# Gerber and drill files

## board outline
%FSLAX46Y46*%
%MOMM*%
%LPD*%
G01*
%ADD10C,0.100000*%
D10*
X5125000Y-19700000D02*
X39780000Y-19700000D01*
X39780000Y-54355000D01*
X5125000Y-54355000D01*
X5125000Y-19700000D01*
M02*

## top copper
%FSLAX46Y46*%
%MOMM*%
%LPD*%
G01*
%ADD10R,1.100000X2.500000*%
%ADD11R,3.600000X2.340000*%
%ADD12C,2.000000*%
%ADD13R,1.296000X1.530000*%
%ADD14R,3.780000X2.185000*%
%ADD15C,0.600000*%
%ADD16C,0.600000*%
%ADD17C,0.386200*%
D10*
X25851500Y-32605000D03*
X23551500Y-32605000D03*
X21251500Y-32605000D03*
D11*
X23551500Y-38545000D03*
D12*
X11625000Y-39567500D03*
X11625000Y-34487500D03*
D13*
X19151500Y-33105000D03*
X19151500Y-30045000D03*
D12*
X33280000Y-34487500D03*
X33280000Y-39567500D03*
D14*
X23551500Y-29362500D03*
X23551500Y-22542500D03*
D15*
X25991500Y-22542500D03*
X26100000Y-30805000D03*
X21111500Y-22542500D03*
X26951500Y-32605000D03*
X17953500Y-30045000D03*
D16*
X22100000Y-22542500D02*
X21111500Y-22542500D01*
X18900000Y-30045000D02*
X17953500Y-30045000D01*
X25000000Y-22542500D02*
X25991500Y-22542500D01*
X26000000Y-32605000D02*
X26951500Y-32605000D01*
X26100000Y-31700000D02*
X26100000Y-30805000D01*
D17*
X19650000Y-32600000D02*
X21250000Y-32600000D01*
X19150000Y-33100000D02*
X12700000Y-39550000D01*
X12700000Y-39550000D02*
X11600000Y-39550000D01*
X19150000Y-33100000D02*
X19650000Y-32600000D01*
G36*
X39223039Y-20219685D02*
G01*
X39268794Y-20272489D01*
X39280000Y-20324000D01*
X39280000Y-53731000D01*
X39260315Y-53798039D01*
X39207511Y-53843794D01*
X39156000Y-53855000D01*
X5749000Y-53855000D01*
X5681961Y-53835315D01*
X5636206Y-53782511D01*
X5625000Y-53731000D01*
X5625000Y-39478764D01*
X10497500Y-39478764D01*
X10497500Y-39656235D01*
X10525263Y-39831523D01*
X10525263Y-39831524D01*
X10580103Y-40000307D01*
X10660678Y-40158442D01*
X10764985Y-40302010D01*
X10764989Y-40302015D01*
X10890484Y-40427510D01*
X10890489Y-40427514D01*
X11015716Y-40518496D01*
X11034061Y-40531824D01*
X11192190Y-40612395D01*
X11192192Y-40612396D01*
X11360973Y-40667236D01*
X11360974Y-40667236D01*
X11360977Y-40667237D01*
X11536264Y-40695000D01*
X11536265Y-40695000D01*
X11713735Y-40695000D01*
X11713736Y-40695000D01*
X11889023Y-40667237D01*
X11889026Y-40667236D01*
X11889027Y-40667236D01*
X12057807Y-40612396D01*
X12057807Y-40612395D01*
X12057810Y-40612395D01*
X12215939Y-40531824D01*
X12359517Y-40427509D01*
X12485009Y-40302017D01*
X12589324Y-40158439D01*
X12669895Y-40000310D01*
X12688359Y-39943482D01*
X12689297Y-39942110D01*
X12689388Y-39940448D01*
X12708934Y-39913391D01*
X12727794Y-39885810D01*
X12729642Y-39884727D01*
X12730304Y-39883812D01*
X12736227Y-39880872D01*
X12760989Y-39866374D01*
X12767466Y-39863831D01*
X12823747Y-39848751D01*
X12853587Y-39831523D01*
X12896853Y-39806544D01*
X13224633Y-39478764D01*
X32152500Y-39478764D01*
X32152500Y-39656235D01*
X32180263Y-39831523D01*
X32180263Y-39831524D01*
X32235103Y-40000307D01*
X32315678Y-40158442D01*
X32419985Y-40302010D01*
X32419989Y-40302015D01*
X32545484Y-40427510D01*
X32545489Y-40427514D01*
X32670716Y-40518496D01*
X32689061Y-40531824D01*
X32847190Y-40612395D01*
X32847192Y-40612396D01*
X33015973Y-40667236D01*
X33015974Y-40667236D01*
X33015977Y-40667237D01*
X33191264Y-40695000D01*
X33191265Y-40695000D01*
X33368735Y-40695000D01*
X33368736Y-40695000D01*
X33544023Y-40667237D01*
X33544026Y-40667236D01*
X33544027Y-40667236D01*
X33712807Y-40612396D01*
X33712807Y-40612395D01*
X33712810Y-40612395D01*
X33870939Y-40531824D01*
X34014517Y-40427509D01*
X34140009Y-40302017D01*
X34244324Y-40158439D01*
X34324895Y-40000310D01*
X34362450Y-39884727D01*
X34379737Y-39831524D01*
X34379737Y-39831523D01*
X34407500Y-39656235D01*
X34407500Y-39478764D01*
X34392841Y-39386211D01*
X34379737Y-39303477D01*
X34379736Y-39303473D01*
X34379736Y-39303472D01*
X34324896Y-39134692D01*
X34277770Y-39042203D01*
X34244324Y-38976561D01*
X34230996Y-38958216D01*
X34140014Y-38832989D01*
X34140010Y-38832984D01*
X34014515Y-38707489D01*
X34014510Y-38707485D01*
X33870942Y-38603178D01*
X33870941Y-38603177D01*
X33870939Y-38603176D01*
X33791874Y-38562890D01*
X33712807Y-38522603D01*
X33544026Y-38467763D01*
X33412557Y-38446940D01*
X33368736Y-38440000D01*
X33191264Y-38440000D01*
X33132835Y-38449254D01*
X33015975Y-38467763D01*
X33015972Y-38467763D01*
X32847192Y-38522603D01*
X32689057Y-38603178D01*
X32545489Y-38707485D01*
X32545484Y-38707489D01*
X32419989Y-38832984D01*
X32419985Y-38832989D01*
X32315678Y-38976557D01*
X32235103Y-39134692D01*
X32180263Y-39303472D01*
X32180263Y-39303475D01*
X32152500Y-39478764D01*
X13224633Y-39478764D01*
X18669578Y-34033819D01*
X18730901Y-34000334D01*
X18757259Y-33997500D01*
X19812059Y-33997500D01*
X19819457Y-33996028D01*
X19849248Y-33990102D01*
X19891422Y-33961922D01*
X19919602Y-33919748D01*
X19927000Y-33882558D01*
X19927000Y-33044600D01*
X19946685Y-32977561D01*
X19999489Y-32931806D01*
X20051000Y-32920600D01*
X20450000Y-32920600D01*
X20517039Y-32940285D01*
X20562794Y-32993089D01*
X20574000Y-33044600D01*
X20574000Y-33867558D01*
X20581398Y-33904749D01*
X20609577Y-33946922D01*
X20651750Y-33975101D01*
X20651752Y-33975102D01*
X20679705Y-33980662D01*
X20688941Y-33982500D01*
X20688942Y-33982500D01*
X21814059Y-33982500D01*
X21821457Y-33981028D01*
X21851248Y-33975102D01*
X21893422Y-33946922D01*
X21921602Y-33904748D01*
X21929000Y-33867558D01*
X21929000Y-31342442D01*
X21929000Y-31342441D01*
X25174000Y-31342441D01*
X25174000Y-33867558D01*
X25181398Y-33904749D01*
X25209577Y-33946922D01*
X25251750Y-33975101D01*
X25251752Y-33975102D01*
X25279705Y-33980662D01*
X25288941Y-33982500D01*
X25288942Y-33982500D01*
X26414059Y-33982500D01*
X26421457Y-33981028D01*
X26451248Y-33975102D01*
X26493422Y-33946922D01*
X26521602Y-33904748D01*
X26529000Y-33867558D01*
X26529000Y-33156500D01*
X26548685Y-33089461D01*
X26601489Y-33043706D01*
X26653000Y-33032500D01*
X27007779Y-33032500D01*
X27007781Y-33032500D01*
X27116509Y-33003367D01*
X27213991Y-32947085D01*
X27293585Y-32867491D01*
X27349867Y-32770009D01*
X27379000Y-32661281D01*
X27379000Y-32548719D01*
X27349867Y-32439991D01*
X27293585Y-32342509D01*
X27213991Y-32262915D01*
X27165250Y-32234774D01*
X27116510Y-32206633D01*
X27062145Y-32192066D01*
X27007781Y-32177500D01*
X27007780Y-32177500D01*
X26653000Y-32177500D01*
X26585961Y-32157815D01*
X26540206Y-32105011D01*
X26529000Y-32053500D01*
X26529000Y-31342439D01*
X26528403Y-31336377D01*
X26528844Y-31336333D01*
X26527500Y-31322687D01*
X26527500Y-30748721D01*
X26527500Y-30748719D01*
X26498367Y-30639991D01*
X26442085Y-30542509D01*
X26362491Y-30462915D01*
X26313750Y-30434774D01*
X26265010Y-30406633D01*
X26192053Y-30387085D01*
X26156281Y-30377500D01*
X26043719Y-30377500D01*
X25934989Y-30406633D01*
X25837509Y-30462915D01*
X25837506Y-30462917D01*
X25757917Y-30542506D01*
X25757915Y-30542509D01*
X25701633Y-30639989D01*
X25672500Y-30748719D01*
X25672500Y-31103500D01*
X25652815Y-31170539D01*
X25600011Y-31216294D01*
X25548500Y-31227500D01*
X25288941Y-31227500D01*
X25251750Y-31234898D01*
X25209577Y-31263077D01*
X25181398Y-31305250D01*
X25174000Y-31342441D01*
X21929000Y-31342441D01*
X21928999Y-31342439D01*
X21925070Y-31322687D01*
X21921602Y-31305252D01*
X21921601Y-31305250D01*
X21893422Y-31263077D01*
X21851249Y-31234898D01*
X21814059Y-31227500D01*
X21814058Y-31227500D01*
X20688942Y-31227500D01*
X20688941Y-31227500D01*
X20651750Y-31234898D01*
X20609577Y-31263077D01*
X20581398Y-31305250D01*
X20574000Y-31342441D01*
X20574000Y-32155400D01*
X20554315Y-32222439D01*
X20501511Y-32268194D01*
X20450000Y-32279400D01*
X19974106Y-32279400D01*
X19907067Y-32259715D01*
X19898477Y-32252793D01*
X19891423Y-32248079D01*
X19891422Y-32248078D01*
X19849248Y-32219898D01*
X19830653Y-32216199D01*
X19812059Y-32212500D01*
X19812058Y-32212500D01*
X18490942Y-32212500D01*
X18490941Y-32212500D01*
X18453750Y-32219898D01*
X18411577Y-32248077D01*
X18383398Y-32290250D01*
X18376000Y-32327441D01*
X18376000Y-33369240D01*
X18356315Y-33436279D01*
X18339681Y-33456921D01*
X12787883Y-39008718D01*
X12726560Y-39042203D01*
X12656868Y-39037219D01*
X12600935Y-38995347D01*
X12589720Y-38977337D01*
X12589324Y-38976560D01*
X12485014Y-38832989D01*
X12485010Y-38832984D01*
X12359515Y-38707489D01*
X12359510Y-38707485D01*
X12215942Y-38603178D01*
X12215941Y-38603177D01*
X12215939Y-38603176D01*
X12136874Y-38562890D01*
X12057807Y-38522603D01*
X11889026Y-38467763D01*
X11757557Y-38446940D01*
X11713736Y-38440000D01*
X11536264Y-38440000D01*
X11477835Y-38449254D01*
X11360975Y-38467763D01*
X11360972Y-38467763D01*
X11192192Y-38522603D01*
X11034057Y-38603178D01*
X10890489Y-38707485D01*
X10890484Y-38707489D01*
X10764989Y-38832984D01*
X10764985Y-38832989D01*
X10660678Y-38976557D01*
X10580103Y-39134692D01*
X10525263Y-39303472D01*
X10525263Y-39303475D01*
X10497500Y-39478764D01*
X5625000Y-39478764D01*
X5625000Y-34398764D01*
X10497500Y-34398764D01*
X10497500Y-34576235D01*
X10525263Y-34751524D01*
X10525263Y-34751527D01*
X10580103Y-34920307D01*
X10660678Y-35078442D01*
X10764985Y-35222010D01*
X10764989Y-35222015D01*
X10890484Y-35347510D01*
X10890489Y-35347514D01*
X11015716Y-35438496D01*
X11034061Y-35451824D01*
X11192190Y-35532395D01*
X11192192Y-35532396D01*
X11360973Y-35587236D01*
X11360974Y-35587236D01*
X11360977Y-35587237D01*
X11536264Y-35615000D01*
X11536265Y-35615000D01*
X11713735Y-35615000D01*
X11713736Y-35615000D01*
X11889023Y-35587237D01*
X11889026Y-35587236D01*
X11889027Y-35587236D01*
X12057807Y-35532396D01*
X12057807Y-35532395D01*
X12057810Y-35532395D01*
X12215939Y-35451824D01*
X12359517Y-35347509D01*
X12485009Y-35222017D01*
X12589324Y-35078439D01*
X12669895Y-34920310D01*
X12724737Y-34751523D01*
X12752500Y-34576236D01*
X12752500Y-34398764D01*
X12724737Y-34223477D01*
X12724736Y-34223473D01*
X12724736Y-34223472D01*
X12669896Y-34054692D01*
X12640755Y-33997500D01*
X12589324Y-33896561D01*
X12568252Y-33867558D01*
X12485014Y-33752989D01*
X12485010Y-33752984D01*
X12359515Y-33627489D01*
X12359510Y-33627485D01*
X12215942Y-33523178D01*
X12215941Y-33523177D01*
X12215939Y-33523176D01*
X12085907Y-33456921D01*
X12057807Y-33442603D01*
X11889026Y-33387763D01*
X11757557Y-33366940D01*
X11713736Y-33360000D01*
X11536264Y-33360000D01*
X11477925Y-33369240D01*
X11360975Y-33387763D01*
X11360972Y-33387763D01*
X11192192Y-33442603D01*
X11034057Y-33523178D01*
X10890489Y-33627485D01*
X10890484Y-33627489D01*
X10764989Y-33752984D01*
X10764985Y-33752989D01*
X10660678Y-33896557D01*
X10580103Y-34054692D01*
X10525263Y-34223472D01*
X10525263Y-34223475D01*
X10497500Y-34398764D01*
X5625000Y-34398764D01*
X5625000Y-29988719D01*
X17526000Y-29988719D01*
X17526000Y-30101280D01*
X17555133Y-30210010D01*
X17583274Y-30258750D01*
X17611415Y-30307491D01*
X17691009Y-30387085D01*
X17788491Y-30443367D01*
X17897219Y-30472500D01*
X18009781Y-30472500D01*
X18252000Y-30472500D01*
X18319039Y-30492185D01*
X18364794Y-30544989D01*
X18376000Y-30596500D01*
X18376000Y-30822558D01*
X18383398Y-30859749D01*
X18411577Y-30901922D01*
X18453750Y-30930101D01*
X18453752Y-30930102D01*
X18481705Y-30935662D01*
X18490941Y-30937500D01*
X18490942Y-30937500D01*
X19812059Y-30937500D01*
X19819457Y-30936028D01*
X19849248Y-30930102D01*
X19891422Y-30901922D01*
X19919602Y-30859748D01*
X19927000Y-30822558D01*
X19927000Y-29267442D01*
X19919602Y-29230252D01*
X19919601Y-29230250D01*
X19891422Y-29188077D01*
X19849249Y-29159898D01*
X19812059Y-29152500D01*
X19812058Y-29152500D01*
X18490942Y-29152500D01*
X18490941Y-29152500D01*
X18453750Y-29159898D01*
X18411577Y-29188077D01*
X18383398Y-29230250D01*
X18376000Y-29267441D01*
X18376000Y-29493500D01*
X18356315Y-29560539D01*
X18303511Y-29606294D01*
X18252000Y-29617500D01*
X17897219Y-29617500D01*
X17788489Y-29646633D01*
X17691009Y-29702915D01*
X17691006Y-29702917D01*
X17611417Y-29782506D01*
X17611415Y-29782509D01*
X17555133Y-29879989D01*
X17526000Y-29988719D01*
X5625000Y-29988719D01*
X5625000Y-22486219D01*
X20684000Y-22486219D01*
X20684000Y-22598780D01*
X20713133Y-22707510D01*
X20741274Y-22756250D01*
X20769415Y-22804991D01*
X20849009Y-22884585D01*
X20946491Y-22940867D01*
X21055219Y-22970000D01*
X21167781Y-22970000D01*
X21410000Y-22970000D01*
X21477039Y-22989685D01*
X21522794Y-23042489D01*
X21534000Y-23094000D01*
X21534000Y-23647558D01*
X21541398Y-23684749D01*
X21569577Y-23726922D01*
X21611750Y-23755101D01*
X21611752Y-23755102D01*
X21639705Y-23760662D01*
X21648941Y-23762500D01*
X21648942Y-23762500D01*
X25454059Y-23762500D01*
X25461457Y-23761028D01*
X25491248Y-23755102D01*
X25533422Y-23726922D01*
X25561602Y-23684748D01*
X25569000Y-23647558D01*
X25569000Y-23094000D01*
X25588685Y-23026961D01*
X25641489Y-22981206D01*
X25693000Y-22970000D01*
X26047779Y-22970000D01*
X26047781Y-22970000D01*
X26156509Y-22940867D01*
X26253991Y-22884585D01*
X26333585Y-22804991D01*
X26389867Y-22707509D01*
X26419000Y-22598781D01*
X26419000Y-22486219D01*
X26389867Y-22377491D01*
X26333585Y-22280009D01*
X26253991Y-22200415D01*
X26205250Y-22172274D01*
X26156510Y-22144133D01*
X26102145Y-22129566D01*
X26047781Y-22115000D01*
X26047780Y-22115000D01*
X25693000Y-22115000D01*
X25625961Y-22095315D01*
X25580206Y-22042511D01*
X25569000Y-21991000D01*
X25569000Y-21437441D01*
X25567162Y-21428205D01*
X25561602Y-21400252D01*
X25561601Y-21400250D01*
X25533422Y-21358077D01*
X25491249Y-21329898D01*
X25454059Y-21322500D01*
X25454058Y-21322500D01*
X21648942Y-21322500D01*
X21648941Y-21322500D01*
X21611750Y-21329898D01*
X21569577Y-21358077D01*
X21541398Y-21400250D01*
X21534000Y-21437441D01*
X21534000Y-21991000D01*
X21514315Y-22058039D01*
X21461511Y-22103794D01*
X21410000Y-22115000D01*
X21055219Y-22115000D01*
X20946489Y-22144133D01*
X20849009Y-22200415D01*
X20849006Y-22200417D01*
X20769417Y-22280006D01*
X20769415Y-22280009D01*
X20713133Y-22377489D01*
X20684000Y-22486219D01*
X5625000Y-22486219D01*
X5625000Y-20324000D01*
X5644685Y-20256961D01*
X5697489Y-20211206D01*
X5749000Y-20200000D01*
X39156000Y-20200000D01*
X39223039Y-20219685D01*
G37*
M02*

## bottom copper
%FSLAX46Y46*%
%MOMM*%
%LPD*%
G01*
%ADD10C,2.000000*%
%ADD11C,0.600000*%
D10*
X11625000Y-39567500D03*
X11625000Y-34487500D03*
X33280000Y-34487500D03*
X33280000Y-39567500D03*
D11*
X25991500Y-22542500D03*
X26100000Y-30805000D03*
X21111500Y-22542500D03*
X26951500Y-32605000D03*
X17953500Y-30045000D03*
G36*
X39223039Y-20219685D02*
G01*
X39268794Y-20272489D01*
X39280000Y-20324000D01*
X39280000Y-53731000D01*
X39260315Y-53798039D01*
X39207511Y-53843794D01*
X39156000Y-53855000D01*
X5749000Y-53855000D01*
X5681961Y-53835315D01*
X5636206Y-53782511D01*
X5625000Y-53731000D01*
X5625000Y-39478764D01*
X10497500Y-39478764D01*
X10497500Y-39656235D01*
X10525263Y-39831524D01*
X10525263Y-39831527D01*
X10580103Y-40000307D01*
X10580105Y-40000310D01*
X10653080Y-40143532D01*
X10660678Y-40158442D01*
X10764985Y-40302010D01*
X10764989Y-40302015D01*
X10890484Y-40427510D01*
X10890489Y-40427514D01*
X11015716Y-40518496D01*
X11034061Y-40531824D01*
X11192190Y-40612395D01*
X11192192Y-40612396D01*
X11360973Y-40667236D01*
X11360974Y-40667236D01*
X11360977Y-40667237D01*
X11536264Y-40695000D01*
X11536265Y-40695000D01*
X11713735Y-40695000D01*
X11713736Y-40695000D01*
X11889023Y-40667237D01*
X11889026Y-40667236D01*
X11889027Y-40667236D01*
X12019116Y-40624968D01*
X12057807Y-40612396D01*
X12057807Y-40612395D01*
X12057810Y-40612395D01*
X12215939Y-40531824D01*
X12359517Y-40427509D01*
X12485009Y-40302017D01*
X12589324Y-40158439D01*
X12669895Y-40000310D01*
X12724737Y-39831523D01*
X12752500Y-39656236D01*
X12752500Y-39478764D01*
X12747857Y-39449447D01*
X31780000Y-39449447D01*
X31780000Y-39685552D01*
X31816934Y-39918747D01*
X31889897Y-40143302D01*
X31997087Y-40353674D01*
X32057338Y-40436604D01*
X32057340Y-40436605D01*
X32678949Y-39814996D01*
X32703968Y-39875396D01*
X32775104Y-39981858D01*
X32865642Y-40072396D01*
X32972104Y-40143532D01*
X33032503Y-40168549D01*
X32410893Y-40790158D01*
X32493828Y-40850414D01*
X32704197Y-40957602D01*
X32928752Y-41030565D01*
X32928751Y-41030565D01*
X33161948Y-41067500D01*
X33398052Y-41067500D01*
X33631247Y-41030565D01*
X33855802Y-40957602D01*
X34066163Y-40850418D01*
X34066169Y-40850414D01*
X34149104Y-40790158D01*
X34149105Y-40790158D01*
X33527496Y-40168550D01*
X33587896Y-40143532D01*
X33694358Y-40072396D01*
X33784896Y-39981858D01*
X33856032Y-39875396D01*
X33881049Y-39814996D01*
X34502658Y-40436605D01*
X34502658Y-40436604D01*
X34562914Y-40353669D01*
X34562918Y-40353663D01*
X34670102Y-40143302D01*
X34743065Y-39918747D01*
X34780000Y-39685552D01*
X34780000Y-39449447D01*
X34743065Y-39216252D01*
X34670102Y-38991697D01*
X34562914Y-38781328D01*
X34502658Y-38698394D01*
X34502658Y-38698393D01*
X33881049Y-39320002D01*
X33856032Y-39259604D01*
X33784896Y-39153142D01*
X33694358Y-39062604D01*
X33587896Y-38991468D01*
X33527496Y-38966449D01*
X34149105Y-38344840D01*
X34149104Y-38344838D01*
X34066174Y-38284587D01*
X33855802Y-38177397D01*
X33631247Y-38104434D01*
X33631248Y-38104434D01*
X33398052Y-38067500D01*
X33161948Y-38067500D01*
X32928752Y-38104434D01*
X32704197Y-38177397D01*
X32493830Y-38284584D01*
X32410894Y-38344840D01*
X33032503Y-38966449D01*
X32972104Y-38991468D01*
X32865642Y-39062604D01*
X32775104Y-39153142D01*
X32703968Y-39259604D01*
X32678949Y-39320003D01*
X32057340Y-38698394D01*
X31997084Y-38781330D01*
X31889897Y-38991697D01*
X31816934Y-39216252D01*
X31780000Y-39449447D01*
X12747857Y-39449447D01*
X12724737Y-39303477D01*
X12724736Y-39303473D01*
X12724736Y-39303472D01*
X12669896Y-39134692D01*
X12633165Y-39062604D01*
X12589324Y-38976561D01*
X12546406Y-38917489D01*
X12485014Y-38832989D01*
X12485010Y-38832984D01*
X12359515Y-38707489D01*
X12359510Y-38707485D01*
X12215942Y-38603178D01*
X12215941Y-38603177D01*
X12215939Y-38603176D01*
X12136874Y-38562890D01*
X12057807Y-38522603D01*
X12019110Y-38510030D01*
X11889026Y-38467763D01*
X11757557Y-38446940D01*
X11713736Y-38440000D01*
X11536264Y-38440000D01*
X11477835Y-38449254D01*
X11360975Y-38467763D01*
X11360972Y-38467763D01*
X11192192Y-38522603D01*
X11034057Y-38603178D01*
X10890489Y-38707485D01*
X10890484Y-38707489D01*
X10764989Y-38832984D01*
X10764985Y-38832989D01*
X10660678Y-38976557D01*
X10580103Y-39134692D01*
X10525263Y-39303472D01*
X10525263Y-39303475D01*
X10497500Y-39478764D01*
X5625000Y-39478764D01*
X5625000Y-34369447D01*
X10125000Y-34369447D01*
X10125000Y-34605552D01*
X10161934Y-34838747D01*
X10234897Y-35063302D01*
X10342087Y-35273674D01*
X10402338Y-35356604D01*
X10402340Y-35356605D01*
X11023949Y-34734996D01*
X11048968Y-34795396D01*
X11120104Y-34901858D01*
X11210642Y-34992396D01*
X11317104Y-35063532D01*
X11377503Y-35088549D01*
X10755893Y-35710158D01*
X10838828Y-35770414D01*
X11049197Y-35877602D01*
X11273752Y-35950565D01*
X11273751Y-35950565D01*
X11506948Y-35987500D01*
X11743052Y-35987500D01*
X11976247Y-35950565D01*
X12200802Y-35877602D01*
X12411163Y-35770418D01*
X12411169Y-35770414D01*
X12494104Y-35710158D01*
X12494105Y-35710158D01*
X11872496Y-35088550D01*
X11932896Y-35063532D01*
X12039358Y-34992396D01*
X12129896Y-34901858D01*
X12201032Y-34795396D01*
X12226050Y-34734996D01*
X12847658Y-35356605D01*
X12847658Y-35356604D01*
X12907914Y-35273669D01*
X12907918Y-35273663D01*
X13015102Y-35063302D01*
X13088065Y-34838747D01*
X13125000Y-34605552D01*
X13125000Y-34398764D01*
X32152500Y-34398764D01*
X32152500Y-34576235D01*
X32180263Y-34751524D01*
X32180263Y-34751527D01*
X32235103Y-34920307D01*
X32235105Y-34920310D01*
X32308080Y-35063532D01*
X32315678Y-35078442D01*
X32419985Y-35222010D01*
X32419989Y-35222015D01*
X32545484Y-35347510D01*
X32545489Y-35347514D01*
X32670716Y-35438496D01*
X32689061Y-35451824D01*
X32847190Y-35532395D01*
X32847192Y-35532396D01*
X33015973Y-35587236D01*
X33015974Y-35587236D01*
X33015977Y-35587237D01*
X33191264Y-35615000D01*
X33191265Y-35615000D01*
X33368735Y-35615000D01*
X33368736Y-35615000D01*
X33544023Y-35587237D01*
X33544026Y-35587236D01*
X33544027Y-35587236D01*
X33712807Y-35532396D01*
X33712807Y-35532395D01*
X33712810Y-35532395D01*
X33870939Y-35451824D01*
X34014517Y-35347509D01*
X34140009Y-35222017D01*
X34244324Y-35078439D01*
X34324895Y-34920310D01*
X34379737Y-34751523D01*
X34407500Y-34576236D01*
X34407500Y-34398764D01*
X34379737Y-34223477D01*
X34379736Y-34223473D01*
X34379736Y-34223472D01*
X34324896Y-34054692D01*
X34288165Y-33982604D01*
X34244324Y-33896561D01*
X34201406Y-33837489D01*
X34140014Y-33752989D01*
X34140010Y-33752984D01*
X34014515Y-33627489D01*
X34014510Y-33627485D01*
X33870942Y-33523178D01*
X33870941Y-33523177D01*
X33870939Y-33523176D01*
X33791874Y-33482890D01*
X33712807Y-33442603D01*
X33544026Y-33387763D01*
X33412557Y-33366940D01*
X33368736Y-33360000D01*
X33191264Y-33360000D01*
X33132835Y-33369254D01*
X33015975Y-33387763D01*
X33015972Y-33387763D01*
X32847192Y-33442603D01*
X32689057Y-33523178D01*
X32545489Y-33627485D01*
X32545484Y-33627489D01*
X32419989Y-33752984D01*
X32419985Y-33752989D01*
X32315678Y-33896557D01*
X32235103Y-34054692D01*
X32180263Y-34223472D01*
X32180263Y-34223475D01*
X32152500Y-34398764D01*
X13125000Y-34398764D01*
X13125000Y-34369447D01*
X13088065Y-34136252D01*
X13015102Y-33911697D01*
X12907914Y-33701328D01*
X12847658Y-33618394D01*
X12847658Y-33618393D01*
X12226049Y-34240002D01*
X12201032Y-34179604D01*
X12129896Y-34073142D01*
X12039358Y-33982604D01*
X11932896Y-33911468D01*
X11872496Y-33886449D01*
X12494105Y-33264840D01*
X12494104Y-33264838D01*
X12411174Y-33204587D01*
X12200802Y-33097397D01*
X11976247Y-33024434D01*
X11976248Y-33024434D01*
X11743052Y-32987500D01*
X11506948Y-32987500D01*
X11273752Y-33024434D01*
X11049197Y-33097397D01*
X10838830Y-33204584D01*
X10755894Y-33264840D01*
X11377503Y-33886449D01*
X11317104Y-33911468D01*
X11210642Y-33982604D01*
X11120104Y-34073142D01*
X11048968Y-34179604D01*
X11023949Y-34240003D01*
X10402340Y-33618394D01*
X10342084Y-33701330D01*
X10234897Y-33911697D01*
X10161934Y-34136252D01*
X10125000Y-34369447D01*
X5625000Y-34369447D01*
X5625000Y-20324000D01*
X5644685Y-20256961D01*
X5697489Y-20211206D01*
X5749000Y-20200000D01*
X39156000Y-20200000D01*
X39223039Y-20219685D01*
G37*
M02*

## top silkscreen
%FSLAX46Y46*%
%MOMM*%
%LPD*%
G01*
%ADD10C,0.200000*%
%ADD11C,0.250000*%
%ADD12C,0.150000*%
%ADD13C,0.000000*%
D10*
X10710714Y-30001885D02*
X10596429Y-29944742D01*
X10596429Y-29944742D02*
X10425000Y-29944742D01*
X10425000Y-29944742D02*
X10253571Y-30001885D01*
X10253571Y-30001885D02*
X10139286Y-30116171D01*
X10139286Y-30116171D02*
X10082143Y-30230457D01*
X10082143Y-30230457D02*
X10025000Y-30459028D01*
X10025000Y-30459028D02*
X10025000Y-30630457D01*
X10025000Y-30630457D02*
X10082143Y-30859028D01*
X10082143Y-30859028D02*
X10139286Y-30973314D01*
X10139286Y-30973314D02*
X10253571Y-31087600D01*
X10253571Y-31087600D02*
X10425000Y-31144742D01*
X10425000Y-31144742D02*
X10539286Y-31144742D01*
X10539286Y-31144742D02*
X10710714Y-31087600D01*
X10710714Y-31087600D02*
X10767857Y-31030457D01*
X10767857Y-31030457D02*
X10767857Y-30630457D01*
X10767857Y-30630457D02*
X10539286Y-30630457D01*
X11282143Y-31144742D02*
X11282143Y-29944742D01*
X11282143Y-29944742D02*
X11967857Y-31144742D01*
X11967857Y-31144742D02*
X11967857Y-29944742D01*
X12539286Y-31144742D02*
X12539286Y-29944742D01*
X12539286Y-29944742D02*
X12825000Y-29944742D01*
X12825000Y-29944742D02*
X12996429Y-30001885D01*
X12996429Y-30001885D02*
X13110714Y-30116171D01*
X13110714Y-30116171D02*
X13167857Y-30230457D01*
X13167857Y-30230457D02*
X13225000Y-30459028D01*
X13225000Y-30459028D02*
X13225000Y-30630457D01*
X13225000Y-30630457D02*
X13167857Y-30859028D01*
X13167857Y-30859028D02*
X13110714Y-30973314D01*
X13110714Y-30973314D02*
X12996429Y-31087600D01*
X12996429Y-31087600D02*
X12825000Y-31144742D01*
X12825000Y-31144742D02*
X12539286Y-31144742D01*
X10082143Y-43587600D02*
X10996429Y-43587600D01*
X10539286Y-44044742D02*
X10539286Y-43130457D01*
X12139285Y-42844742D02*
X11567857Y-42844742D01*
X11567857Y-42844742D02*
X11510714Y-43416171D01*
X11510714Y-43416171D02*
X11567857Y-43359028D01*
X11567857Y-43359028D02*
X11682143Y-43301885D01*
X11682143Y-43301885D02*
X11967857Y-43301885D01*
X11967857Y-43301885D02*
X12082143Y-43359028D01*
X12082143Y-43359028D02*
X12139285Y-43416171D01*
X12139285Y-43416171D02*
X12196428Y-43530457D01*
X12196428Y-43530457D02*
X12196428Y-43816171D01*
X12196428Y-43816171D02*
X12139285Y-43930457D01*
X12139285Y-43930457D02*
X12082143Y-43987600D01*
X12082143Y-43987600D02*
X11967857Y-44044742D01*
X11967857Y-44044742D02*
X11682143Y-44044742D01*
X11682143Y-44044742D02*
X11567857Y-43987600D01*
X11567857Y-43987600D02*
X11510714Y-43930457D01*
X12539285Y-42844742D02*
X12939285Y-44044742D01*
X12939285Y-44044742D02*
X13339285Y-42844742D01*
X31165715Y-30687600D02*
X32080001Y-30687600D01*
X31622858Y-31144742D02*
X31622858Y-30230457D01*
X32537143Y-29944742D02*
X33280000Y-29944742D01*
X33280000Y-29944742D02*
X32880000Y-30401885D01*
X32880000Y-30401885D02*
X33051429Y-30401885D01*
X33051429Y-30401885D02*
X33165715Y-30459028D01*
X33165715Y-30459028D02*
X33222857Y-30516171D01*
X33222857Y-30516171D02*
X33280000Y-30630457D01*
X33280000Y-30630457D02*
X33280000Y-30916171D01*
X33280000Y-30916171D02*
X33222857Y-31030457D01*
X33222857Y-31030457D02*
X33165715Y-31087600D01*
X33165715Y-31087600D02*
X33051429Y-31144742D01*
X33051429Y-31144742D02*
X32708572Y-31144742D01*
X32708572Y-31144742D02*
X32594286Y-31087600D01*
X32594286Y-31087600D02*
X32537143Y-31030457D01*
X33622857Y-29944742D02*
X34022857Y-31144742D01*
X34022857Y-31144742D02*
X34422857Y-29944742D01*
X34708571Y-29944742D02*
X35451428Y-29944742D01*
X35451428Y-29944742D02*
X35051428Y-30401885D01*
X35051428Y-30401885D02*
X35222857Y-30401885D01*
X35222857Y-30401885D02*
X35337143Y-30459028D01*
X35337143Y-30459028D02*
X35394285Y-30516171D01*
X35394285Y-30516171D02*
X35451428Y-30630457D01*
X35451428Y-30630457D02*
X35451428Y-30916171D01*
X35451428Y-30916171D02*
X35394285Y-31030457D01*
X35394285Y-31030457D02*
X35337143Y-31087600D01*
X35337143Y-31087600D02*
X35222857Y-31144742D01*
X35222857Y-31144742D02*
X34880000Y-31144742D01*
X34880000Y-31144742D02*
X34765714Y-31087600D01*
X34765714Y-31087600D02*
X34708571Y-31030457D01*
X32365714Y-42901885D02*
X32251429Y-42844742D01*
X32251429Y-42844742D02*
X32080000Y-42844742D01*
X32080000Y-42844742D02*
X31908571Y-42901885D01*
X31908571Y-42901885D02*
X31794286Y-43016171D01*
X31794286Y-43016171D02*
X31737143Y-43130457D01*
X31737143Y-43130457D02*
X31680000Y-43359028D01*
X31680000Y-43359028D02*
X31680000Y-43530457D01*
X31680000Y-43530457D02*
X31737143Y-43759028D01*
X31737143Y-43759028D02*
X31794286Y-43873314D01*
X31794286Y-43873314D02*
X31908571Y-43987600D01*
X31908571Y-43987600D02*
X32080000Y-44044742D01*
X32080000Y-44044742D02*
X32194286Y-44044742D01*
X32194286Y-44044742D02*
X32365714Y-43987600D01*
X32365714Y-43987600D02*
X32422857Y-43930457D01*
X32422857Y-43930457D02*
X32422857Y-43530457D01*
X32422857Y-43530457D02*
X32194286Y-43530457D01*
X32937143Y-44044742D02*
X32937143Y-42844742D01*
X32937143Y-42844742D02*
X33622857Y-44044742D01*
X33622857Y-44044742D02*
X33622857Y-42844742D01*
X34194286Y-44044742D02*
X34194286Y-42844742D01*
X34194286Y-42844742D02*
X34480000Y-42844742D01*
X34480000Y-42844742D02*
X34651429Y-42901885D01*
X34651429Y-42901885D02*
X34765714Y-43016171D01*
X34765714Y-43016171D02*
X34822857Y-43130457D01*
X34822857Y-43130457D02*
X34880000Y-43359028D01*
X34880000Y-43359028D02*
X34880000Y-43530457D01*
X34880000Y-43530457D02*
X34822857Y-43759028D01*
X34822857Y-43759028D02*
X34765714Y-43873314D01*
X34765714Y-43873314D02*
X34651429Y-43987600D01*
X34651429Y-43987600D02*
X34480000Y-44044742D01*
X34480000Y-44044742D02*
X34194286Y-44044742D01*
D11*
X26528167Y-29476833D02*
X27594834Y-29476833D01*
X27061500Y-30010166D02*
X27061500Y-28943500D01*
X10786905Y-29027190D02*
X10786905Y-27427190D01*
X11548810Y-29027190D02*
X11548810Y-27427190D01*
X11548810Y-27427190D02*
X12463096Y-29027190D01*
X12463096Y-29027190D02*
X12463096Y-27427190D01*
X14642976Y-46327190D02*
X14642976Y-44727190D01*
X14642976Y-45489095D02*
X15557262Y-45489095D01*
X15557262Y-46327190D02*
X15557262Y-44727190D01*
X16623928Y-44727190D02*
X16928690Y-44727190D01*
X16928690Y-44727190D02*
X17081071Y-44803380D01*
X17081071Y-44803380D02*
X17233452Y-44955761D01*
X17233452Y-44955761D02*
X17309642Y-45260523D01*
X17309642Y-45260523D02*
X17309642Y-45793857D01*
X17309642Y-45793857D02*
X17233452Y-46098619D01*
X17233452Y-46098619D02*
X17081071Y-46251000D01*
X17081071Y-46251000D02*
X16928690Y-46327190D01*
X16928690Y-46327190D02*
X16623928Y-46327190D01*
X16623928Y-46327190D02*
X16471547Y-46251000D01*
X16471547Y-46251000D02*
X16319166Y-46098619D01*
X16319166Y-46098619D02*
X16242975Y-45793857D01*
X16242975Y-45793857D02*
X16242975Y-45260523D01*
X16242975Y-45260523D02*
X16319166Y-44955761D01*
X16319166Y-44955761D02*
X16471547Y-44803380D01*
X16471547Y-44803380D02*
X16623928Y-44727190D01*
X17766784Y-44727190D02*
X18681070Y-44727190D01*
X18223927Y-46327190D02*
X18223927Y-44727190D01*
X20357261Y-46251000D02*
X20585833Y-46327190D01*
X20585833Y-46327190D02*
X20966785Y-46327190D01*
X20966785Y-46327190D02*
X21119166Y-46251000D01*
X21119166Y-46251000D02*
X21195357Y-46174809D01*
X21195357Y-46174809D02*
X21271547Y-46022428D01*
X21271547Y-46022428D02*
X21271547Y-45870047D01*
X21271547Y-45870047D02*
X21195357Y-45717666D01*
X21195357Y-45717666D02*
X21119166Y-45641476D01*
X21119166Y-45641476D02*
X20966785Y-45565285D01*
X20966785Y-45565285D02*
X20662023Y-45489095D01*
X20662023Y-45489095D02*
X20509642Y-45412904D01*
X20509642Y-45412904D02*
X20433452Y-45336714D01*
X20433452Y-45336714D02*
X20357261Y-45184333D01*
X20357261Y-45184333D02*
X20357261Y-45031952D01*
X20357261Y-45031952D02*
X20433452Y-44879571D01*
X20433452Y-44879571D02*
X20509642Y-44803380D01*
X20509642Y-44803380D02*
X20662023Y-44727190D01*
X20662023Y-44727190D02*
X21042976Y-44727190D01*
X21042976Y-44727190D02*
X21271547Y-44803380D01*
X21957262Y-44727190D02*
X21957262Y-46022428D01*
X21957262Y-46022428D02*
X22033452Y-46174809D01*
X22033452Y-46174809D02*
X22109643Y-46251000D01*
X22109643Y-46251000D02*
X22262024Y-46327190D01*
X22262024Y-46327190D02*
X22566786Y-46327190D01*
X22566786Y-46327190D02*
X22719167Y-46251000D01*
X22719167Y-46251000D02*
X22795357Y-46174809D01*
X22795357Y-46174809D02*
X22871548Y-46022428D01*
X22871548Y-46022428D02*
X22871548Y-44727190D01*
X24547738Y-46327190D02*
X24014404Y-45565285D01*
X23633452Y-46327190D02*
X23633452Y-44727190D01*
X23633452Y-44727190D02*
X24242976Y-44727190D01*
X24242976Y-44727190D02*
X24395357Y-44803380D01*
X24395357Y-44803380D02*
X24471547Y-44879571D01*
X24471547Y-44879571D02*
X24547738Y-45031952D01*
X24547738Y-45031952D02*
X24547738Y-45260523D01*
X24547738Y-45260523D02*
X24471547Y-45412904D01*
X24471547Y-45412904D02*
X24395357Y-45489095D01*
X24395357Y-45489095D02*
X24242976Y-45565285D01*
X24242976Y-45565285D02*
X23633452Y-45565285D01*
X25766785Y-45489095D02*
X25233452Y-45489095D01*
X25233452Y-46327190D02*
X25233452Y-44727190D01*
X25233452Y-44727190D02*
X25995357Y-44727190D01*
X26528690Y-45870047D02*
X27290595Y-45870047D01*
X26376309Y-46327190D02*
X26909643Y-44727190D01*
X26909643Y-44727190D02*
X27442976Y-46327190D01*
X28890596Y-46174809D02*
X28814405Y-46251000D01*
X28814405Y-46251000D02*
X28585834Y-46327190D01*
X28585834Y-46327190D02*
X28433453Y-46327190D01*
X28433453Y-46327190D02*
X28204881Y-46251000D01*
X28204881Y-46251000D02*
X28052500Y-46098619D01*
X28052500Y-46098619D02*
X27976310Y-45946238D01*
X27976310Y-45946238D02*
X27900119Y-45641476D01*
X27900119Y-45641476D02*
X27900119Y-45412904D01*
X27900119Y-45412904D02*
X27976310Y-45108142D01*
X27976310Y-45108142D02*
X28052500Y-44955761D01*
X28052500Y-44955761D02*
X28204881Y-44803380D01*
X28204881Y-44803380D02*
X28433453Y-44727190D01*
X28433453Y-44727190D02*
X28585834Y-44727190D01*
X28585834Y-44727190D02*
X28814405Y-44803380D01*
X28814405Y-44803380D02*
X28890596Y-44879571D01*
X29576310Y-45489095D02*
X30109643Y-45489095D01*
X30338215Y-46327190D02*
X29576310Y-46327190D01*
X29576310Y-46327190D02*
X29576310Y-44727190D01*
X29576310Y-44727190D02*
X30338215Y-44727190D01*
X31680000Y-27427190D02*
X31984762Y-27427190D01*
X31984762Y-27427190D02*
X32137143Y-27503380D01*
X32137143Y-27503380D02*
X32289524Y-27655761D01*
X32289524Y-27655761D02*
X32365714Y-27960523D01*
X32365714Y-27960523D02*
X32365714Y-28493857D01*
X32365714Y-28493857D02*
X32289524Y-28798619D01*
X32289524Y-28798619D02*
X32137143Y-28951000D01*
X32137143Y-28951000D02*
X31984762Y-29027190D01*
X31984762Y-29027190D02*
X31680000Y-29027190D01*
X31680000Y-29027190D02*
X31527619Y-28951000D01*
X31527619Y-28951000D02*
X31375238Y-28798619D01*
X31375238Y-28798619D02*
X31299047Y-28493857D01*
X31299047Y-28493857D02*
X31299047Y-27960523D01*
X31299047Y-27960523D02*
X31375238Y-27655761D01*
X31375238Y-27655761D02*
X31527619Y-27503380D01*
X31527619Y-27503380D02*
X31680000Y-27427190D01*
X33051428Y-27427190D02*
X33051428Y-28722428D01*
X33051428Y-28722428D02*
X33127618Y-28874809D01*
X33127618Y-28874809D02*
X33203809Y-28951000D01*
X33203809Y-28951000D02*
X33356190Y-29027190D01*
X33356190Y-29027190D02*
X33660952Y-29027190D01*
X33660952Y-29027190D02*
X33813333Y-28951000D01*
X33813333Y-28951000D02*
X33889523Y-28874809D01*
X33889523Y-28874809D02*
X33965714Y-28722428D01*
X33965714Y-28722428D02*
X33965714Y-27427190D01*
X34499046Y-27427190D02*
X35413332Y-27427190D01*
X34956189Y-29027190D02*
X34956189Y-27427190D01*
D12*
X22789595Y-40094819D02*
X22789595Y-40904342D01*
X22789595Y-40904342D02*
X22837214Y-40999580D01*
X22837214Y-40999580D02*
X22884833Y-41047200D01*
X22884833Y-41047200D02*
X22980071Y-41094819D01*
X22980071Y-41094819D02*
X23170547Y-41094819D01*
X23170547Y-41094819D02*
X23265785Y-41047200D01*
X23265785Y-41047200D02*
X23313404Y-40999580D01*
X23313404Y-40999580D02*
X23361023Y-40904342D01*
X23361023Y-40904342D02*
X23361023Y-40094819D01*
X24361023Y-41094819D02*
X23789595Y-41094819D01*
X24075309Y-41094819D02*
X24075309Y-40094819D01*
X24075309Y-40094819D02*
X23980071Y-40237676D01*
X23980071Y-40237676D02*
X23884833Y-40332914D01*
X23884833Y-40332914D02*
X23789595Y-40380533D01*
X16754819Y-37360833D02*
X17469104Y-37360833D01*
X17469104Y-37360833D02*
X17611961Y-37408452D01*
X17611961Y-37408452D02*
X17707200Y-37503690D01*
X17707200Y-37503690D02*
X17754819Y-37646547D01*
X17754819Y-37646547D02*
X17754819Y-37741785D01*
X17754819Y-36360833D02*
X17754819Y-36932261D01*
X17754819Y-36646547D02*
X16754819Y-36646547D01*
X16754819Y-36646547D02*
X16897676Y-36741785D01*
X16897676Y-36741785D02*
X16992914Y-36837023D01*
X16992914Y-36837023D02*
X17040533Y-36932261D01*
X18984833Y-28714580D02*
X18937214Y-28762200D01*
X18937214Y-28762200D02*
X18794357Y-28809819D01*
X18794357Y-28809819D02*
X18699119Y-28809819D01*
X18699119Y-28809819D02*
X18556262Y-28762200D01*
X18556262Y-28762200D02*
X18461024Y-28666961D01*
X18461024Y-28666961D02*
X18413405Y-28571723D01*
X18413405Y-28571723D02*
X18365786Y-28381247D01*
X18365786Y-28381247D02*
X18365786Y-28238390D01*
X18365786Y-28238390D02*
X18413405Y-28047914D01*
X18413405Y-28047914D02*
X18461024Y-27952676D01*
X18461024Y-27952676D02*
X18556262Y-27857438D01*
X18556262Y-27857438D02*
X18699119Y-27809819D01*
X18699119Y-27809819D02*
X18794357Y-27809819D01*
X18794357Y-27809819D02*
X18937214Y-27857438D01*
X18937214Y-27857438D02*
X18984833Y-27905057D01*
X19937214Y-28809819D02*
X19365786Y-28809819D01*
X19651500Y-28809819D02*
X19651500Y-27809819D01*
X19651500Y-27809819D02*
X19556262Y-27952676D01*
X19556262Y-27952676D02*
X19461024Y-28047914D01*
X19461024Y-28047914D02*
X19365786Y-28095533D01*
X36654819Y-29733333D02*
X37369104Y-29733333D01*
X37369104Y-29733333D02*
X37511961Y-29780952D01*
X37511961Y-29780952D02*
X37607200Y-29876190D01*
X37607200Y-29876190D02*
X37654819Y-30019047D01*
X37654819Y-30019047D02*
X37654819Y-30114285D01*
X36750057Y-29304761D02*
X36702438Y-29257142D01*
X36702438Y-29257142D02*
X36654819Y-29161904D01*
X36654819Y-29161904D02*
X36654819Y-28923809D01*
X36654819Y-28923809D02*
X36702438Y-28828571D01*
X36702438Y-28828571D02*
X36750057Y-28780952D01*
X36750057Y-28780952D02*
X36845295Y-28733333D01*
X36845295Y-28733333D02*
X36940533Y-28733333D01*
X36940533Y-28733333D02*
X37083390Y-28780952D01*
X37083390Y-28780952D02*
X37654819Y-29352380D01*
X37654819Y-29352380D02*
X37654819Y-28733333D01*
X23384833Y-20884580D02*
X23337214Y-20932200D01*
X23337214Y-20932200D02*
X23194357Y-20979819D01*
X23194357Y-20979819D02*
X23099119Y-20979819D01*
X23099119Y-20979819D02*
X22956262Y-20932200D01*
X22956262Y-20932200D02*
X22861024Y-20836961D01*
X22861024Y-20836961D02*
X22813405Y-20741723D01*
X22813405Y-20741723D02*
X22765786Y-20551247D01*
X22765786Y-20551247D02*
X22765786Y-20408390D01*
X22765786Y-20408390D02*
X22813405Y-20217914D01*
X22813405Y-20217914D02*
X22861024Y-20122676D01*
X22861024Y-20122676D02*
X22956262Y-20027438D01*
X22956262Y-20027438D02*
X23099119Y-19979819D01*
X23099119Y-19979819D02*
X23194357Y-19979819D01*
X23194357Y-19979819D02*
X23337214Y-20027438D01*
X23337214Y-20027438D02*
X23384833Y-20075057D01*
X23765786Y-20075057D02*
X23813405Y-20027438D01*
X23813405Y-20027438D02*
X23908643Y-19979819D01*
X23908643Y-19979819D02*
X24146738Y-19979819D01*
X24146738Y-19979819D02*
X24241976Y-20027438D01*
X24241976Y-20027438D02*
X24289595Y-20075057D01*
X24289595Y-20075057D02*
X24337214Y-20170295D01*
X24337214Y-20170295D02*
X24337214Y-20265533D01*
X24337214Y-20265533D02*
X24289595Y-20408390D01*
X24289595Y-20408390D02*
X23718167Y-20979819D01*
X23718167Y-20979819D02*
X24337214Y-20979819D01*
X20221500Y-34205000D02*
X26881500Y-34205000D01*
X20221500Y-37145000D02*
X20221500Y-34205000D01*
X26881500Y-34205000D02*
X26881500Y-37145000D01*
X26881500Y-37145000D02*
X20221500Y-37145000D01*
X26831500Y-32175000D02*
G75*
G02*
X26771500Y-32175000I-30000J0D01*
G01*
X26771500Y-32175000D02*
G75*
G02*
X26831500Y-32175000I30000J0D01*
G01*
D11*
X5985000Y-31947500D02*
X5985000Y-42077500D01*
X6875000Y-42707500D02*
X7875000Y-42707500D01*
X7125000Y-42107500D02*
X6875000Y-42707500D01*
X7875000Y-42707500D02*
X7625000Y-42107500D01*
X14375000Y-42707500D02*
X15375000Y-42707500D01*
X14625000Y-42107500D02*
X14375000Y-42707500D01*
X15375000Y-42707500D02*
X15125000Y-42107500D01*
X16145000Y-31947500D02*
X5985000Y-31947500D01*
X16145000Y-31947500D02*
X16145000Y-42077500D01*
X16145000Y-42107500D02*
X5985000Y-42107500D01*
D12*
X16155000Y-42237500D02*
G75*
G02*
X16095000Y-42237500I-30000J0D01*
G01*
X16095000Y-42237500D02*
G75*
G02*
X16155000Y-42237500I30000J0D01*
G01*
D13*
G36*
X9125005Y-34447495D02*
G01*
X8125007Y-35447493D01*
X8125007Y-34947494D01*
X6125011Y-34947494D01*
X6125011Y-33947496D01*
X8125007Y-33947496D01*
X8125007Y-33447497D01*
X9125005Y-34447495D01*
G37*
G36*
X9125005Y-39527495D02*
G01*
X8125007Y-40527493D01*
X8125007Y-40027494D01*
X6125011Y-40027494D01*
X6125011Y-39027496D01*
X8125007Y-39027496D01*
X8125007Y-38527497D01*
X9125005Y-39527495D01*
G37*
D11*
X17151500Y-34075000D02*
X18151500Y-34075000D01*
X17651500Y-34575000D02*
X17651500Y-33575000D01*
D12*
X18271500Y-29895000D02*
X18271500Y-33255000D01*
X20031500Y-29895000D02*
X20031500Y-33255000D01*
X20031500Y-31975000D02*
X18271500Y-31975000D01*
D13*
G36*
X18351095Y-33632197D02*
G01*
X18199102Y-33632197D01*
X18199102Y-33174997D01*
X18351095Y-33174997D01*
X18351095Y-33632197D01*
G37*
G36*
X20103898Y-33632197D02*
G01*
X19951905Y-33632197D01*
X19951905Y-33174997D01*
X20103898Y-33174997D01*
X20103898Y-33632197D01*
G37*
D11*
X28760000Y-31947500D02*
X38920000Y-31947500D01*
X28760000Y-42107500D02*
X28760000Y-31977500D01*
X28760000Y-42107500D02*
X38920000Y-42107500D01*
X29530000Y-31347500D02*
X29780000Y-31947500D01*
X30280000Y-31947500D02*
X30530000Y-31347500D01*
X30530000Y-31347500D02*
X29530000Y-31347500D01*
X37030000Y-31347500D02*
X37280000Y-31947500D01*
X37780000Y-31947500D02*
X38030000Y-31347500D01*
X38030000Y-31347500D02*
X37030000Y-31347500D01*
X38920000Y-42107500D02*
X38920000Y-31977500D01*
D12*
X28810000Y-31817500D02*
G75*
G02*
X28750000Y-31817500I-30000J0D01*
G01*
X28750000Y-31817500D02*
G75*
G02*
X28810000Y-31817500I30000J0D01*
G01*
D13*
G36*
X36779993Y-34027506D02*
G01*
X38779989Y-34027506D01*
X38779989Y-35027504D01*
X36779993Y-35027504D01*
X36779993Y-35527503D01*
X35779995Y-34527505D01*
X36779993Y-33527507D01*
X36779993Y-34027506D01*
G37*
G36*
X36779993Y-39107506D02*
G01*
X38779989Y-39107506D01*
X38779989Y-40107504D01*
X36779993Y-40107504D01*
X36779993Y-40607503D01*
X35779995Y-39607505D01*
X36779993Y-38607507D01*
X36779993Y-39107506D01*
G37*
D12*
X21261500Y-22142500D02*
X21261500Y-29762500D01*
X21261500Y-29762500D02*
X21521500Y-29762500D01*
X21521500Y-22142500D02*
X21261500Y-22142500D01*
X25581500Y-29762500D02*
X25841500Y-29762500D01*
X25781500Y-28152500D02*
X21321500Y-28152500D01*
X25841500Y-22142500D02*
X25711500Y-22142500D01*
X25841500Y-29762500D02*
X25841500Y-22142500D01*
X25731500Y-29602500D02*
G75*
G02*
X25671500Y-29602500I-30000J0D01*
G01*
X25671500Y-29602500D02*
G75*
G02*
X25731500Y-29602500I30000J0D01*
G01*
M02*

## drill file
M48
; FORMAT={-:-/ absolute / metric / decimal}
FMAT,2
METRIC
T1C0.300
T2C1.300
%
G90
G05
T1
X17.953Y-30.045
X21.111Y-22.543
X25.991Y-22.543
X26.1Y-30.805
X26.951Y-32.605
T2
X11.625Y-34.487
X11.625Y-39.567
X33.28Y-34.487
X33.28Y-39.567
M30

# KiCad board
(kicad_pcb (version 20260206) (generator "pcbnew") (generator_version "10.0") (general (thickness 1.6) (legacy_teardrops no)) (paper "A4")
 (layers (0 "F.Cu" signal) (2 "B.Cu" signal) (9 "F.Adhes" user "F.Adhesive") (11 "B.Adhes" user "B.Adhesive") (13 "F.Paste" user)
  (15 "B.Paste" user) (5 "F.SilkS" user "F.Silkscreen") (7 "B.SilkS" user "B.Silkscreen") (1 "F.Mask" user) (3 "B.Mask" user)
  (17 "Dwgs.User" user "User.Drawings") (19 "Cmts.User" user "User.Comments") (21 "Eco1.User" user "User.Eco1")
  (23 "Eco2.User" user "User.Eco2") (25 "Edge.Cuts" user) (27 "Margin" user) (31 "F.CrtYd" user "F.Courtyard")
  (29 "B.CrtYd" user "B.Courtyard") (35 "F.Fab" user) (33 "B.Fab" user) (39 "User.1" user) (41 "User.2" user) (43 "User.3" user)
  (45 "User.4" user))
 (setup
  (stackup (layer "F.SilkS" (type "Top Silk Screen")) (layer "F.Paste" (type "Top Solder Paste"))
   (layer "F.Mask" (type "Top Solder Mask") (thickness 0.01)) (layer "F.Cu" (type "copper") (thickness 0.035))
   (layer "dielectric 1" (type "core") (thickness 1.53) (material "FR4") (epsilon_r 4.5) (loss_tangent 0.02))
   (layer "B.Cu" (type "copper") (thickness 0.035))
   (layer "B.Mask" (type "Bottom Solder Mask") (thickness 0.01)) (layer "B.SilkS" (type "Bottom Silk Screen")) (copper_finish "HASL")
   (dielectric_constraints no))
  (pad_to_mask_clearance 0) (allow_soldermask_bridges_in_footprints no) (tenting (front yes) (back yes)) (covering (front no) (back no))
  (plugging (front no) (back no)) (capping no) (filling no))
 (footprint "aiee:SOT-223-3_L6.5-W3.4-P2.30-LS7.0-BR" (layer "F.Cu") (at 23.5515 35.575 90)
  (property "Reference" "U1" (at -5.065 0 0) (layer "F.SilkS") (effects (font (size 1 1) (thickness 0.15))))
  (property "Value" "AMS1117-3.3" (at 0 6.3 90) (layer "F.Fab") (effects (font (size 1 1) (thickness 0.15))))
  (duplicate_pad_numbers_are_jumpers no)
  (fp_line (start 1.37 -3.33) (end 1.37 3.33) (stroke (width 0.15) (type solid)) (layer "F.SilkS"))
  (fp_line (start -1.57 -3.33) (end 1.37 -3.33) (stroke (width 0.15) (type solid)) (layer "F.SilkS"))
  (fp_line (start 1.37 3.33) (end -1.57 3.33) (stroke (width 0.15) (type solid)) (layer "F.SilkS"))
  (fp_line (start -1.57 3.33) (end -1.57 -3.33) (stroke (width 0.15) (type solid)) (layer "F.SilkS"))
  (fp_circle (center 3.4 3.25) (end 3.43 3.25) (stroke (width 0.15) (type solid)) (fill no) (layer "F.SilkS"))
  (pad "1" smd rect (at 2.97 2.3 90) (size 2.5 1.1) (layers "F.Cu" "F.Mask" "F.Paste") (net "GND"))
  (pad "2" smd rect (at 2.97 0 90) (size 2.5 1.1) (layers "F.Cu" "F.Mask" "F.Paste") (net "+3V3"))
  (pad "3" smd rect (at 2.97 -2.3 90) (size 2.5 1.1) (layers "F.Cu" "F.Mask" "F.Paste") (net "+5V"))
  (pad "4" smd rect (at -2.97 0 90) (size 2.34 3.6) (layers "F.Cu" "F.Mask" "F.Paste") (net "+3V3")))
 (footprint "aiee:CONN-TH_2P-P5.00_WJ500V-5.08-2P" (layer "F.Cu") (at 11.625 37.0275 90)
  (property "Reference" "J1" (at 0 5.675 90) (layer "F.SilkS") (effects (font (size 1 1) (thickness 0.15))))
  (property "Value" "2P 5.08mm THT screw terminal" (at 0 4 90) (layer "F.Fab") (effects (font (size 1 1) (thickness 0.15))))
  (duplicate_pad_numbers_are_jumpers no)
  (fp_line (start 5.08 -5.64) (end -5.05 -5.64) (stroke (width 0.25) (type solid)) (layer "F.SilkS"))
  (fp_line (start -5.68 -4.75) (end -5.68 -3.75) (stroke (width 0.25) (type solid)) (layer "F.SilkS"))
  (fp_line (start -5.08 -4.5) (end -5.68 -4.75) (stroke (width 0.25) (type solid)) (layer "F.SilkS"))
  (fp_line (start -5.68 -3.75) (end -5.08 -4) (stroke (width 0.25) (type solid)) (layer "F.SilkS"))
  (fp_line (start -5.68 2.75) (end -5.68 3.75) (stroke (width 0.25) (type solid)) (layer "F.SilkS"))
  (fp_line (start -5.08 3) (end -5.68 2.75) (stroke (width 0.25) (type solid)) (layer "F.SilkS"))
  (fp_line (start -5.68 3.75) (end -5.08 3.5) (stroke (width 0.25) (type solid)) (layer "F.SilkS"))
  (fp_line (start 5.08 4.52) (end 5.08 -5.64) (stroke (width 0.25) (type solid)) (layer "F.SilkS"))
  (fp_line (start 5.08 4.52) (end -5.05 4.52) (stroke (width 0.25) (type solid)) (layer "F.SilkS"))
  (fp_line (start -5.08 4.52) (end -5.08 -5.64) (stroke (width 0.25) (type solid)) (layer "F.SilkS"))
  (fp_circle (center -5.21 4.5) (end -5.18 4.5) (stroke (width 0.15) (type solid)) (fill no) (layer "F.SilkS"))
  (fp_poly
   (pts (xy 2.080006 -5.499989) (xy 3.080004 -5.499989) (xy 3.080004 -3.499993) (xy 3.580003 -3.499993) (xy 2.580005 -2.499995)
    (xy 1.580007 -3.499993) (xy 2.080006 -3.499993) (xy 2.080006 -5.499989))
   (stroke (width 0) (type solid)) (fill yes) (layer "F.SilkS"))
  (fp_poly
   (pts (xy -2.999994 -5.499989) (xy -1.999996 -5.499989) (xy -1.999996 -3.499993) (xy -1.499997 -3.499993) (xy -2.499995 -2.499995)
    (xy -3.499993 -3.499993) (xy -2.999994 -3.499993) (xy -2.999994 -5.499989))
   (stroke (width 0) (type solid)) (fill yes) (layer "F.SilkS"))
  (pad "1" thru_hole circle (at -2.54 0 270) (size 2 2) (drill 1.300022) (layers "*.Cu" "*.Mask") (remove_unused_layers no) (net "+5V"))
  (pad "2" thru_hole circle (at 2.54 0 270) (size 2 2) (drill 1.300022) (layers "*.Cu" "*.Mask") (remove_unused_layers no) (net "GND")))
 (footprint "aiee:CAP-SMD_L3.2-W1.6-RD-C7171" (layer "F.Cu") (at 19.1515 31.575 90)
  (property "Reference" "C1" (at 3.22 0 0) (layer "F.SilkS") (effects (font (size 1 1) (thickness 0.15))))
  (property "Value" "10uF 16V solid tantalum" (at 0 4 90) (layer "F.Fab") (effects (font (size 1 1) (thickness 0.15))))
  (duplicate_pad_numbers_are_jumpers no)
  (fp_line (start -2.5 -2) (end -2.5 -1) (stroke (width 0.25) (type solid)) (layer "F.SilkS"))
  (fp_line (start -3 -1.5) (end -2 -1.5) (stroke (width 0.25) (type solid)) (layer "F.SilkS"))
  (fp_line (start 1.68 -0.88) (end -1.68 -0.88) (stroke (width 0.15) (type solid)) (layer "F.SilkS"))
  (fp_line (start 1.68 0.88) (end -1.68 0.88) (stroke (width 0.15) (type solid)) (layer "F.SilkS"))
  (fp_line (start -0.4 0.88) (end -0.4 -0.88) (stroke (width 0.15) (type solid)) (layer "F.SilkS"))
  (fp_poly
   (pts (xy -1.599997 -0.952398) (xy -1.599997 -0.800405) (xy -2.057197 -0.800405) (xy -2.057197 -0.952398) (xy -1.599997 -0.952398))
   (stroke (width 0) (type solid)) (fill yes) (layer "F.SilkS"))
  (fp_poly
   (pts (xy -1.599997 0.952398) (xy -1.599997 0.800405) (xy -2.057197 0.800405) (xy -2.057197 0.952398) (xy -1.599997 0.952398))
   (stroke (width 0) (type solid)) (fill yes) (layer "F.SilkS"))
  (pad "1" smd rect (at -1.53 0 270) (size 1.53 1.296) (layers "F.Cu" "F.Mask" "F.Paste") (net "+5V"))
  (pad "2" smd rect (at 1.53 0 270) (size 1.53 1.296) (layers "F.Cu" "F.Mask" "F.Paste") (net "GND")))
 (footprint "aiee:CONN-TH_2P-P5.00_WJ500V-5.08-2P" (layer "F.Cu") (at 33.28 37.0275 -90)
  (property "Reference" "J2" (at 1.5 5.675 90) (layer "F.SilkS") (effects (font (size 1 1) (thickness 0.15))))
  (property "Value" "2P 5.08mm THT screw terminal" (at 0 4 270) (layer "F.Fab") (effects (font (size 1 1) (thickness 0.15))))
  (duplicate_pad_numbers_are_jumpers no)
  (fp_line (start -5.08 4.52) (end -5.08 -5.64) (stroke (width 0.25) (type solid)) (layer "F.SilkS"))
  (fp_line (start 5.08 4.52) (end -5.05 4.52) (stroke (width 0.25) (type solid)) (layer "F.SilkS"))
  (fp_line (start 5.08 4.52) (end 5.08 -5.64) (stroke (width 0.25) (type solid)) (layer "F.SilkS"))
  (fp_line (start -5.68 3.75) (end -5.08 3.5) (stroke (width 0.25) (type solid)) (layer "F.SilkS"))
  (fp_line (start -5.08 3) (end -5.68 2.75) (stroke (width 0.25) (type solid)) (layer "F.SilkS"))
  (fp_line (start -5.68 2.75) (end -5.68 3.75) (stroke (width 0.25) (type solid)) (layer "F.SilkS"))
  (fp_line (start -5.68 -3.75) (end -5.08 -4) (stroke (width 0.25) (type solid)) (layer "F.SilkS"))
  (fp_line (start -5.08 -4.5) (end -5.68 -4.75) (stroke (width 0.25) (type solid)) (layer "F.SilkS"))
  (fp_line (start -5.68 -4.75) (end -5.68 -3.75) (stroke (width 0.25) (type solid)) (layer "F.SilkS"))
  (fp_line (start 5.08 -5.64) (end -5.05 -5.64) (stroke (width 0.25) (type solid)) (layer "F.SilkS"))
  (fp_circle (center -5.21 4.5) (end -5.18 4.5) (stroke (width 0.15) (type solid)) (fill no) (layer "F.SilkS"))
  (fp_poly
   (pts (xy -2.999994 -5.499989) (xy -1.999996 -5.499989) (xy -1.999996 -3.499993) (xy -1.499997 -3.499993) (xy -2.499995 -2.499995)
    (xy -3.499993 -3.499993) (xy -2.999994 -3.499993) (xy -2.999994 -5.499989))
   (stroke (width 0) (type solid)) (fill yes) (layer "F.SilkS"))
  (fp_poly
   (pts (xy 2.080006 -5.499989) (xy 3.080004 -5.499989) (xy 3.080004 -3.499993) (xy 3.580003 -3.499993) (xy 2.580005 -2.499995)
    (xy 1.580007 -3.499993) (xy 2.080006 -3.499993) (xy 2.080006 -5.499989))
   (stroke (width 0) (type solid)) (fill yes) (layer "F.SilkS"))
  (pad "1" thru_hole circle (at -2.54 0 90) (size 2 2) (drill 1.300022) (layers "*.Cu" "*.Mask") (remove_unused_layers no) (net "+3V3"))
  (pad "2" thru_hole circle (at 2.54 0 90) (size 2 2) (drill 1.300022) (layers "*.Cu" "*.Mask") (remove_unused_layers no) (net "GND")))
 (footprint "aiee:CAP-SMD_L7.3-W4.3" (layer "F.Cu") (at 23.5515 25.9525 -90)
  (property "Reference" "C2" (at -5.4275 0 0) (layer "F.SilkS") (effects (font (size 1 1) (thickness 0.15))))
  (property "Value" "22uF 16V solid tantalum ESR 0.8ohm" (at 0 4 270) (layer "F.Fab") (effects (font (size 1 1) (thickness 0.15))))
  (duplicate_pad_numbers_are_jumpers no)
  (fp_line (start -3.81 2.29) (end 3.81 2.29) (stroke (width 0.15) (type solid)) (layer "F.SilkS"))
  (fp_line (start 3.81 2.29) (end 3.81 2.03) (stroke (width 0.15) (type solid)) (layer "F.SilkS"))
  (fp_line (start -3.81 2.03) (end -3.81 2.29) (stroke (width 0.15) (type solid)) (layer "F.SilkS"))
  (fp_line (start 3.81 -2.03) (end 3.81 -2.29) (stroke (width 0.15) (type solid)) (layer "F.SilkS"))
  (fp_line (start 2.2 -2.23) (end 2.2 2.23) (stroke (width 0.15) (type solid)) (layer "F.SilkS"))
  (fp_line (start -3.81 -2.29) (end -3.81 -2.16) (stroke (width 0.15) (type solid)) (layer "F.SilkS"))
  (fp_line (start 3.81 -2.29) (end -3.81 -2.29) (stroke (width 0.15) (type solid)) (layer "F.SilkS"))
  (fp_circle (center 3.65 -2.15) (end 3.68 -2.15) (stroke (width 0.15) (type solid)) (fill no) (layer "F.SilkS"))
  (pad "1" smd rect (at 3.41 0 90) (size 2.185 3.78) (layers "F.Cu" "F.Mask" "F.Paste") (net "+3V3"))
  (pad "2" smd rect (at -3.41 0 90) (size 2.185 3.78) (layers "F.Cu" "F.Mask" "F.Paste") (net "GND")))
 (gr_rect (start 5.125 19.7) (end 39.78 54.355) (stroke (width 0.1) (type default)) (fill no) (layer "Edge.Cuts"))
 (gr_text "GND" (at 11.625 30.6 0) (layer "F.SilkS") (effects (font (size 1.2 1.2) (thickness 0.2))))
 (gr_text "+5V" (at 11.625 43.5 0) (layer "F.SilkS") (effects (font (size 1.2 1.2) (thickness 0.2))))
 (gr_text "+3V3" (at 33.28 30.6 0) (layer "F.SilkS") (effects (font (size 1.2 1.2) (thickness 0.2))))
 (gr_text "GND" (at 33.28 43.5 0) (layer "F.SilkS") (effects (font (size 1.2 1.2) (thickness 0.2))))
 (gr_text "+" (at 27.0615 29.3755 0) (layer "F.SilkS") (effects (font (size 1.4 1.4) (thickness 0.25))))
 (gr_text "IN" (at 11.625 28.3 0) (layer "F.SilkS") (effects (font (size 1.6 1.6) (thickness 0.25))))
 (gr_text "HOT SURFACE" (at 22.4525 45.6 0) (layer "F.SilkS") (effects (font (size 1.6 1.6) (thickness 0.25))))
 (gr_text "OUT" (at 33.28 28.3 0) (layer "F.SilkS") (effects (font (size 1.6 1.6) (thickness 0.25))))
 (segment (start 22.1 22.5425) (end 21.1115 22.5425) (width 0.6) (layer "F.Cu") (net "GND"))
 (segment (start 18.9 30.045) (end 17.9535 30.045) (width 0.6) (layer "F.Cu") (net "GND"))
 (segment (start 25 22.5425) (end 25.9915 22.5425) (width 0.6) (layer "F.Cu") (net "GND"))
 (segment (start 26 32.605) (end 26.9515 32.605) (width 0.6) (layer "F.Cu") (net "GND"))
 (segment (start 26.1 31.7) (end 26.1 30.805) (width 0.6) (layer "F.Cu") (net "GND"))
 (via (at 25.9915 22.5425) (size 0.6) (drill 0.3) (layers "F.Cu" "B.Cu") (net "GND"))
 (via (at 26.1 30.805) (size 0.6) (drill 0.3) (layers "F.Cu" "B.Cu") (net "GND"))
 (via (at 21.1115 22.5425) (size 0.6) (drill 0.3) (layers "F.Cu" "B.Cu") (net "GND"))
 (via (at 26.9515 32.605) (size 0.6) (drill 0.3) (layers "F.Cu" "B.Cu") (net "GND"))
 (via (at 17.9535 30.045) (size 0.6) (drill 0.3) (layers "F.Cu" "B.Cu") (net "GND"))
 (segment (start 19.65 32.6) (end 21.25 32.6) (width 0.3862) (layer "F.Cu") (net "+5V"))
 (segment (start 19.15 33.1) (end 12.7 39.55) (width 0.3862) (layer "F.Cu") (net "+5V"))
 (segment (start 12.7 39.55) (end 11.6 39.55) (width 0.3862) (layer "F.Cu") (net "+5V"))
 (segment (start 19.15 33.1) (end 19.65 32.6) (width 0.3862) (layer "F.Cu") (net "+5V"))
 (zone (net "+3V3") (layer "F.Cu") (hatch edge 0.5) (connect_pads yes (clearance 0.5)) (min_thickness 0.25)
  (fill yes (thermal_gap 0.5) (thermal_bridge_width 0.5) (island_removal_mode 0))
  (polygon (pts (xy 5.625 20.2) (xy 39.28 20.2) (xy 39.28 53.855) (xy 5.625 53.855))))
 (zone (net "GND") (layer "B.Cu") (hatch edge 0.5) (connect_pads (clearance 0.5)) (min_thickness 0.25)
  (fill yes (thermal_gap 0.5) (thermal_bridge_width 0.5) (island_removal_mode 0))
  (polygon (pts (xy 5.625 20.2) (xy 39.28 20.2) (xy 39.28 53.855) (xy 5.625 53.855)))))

